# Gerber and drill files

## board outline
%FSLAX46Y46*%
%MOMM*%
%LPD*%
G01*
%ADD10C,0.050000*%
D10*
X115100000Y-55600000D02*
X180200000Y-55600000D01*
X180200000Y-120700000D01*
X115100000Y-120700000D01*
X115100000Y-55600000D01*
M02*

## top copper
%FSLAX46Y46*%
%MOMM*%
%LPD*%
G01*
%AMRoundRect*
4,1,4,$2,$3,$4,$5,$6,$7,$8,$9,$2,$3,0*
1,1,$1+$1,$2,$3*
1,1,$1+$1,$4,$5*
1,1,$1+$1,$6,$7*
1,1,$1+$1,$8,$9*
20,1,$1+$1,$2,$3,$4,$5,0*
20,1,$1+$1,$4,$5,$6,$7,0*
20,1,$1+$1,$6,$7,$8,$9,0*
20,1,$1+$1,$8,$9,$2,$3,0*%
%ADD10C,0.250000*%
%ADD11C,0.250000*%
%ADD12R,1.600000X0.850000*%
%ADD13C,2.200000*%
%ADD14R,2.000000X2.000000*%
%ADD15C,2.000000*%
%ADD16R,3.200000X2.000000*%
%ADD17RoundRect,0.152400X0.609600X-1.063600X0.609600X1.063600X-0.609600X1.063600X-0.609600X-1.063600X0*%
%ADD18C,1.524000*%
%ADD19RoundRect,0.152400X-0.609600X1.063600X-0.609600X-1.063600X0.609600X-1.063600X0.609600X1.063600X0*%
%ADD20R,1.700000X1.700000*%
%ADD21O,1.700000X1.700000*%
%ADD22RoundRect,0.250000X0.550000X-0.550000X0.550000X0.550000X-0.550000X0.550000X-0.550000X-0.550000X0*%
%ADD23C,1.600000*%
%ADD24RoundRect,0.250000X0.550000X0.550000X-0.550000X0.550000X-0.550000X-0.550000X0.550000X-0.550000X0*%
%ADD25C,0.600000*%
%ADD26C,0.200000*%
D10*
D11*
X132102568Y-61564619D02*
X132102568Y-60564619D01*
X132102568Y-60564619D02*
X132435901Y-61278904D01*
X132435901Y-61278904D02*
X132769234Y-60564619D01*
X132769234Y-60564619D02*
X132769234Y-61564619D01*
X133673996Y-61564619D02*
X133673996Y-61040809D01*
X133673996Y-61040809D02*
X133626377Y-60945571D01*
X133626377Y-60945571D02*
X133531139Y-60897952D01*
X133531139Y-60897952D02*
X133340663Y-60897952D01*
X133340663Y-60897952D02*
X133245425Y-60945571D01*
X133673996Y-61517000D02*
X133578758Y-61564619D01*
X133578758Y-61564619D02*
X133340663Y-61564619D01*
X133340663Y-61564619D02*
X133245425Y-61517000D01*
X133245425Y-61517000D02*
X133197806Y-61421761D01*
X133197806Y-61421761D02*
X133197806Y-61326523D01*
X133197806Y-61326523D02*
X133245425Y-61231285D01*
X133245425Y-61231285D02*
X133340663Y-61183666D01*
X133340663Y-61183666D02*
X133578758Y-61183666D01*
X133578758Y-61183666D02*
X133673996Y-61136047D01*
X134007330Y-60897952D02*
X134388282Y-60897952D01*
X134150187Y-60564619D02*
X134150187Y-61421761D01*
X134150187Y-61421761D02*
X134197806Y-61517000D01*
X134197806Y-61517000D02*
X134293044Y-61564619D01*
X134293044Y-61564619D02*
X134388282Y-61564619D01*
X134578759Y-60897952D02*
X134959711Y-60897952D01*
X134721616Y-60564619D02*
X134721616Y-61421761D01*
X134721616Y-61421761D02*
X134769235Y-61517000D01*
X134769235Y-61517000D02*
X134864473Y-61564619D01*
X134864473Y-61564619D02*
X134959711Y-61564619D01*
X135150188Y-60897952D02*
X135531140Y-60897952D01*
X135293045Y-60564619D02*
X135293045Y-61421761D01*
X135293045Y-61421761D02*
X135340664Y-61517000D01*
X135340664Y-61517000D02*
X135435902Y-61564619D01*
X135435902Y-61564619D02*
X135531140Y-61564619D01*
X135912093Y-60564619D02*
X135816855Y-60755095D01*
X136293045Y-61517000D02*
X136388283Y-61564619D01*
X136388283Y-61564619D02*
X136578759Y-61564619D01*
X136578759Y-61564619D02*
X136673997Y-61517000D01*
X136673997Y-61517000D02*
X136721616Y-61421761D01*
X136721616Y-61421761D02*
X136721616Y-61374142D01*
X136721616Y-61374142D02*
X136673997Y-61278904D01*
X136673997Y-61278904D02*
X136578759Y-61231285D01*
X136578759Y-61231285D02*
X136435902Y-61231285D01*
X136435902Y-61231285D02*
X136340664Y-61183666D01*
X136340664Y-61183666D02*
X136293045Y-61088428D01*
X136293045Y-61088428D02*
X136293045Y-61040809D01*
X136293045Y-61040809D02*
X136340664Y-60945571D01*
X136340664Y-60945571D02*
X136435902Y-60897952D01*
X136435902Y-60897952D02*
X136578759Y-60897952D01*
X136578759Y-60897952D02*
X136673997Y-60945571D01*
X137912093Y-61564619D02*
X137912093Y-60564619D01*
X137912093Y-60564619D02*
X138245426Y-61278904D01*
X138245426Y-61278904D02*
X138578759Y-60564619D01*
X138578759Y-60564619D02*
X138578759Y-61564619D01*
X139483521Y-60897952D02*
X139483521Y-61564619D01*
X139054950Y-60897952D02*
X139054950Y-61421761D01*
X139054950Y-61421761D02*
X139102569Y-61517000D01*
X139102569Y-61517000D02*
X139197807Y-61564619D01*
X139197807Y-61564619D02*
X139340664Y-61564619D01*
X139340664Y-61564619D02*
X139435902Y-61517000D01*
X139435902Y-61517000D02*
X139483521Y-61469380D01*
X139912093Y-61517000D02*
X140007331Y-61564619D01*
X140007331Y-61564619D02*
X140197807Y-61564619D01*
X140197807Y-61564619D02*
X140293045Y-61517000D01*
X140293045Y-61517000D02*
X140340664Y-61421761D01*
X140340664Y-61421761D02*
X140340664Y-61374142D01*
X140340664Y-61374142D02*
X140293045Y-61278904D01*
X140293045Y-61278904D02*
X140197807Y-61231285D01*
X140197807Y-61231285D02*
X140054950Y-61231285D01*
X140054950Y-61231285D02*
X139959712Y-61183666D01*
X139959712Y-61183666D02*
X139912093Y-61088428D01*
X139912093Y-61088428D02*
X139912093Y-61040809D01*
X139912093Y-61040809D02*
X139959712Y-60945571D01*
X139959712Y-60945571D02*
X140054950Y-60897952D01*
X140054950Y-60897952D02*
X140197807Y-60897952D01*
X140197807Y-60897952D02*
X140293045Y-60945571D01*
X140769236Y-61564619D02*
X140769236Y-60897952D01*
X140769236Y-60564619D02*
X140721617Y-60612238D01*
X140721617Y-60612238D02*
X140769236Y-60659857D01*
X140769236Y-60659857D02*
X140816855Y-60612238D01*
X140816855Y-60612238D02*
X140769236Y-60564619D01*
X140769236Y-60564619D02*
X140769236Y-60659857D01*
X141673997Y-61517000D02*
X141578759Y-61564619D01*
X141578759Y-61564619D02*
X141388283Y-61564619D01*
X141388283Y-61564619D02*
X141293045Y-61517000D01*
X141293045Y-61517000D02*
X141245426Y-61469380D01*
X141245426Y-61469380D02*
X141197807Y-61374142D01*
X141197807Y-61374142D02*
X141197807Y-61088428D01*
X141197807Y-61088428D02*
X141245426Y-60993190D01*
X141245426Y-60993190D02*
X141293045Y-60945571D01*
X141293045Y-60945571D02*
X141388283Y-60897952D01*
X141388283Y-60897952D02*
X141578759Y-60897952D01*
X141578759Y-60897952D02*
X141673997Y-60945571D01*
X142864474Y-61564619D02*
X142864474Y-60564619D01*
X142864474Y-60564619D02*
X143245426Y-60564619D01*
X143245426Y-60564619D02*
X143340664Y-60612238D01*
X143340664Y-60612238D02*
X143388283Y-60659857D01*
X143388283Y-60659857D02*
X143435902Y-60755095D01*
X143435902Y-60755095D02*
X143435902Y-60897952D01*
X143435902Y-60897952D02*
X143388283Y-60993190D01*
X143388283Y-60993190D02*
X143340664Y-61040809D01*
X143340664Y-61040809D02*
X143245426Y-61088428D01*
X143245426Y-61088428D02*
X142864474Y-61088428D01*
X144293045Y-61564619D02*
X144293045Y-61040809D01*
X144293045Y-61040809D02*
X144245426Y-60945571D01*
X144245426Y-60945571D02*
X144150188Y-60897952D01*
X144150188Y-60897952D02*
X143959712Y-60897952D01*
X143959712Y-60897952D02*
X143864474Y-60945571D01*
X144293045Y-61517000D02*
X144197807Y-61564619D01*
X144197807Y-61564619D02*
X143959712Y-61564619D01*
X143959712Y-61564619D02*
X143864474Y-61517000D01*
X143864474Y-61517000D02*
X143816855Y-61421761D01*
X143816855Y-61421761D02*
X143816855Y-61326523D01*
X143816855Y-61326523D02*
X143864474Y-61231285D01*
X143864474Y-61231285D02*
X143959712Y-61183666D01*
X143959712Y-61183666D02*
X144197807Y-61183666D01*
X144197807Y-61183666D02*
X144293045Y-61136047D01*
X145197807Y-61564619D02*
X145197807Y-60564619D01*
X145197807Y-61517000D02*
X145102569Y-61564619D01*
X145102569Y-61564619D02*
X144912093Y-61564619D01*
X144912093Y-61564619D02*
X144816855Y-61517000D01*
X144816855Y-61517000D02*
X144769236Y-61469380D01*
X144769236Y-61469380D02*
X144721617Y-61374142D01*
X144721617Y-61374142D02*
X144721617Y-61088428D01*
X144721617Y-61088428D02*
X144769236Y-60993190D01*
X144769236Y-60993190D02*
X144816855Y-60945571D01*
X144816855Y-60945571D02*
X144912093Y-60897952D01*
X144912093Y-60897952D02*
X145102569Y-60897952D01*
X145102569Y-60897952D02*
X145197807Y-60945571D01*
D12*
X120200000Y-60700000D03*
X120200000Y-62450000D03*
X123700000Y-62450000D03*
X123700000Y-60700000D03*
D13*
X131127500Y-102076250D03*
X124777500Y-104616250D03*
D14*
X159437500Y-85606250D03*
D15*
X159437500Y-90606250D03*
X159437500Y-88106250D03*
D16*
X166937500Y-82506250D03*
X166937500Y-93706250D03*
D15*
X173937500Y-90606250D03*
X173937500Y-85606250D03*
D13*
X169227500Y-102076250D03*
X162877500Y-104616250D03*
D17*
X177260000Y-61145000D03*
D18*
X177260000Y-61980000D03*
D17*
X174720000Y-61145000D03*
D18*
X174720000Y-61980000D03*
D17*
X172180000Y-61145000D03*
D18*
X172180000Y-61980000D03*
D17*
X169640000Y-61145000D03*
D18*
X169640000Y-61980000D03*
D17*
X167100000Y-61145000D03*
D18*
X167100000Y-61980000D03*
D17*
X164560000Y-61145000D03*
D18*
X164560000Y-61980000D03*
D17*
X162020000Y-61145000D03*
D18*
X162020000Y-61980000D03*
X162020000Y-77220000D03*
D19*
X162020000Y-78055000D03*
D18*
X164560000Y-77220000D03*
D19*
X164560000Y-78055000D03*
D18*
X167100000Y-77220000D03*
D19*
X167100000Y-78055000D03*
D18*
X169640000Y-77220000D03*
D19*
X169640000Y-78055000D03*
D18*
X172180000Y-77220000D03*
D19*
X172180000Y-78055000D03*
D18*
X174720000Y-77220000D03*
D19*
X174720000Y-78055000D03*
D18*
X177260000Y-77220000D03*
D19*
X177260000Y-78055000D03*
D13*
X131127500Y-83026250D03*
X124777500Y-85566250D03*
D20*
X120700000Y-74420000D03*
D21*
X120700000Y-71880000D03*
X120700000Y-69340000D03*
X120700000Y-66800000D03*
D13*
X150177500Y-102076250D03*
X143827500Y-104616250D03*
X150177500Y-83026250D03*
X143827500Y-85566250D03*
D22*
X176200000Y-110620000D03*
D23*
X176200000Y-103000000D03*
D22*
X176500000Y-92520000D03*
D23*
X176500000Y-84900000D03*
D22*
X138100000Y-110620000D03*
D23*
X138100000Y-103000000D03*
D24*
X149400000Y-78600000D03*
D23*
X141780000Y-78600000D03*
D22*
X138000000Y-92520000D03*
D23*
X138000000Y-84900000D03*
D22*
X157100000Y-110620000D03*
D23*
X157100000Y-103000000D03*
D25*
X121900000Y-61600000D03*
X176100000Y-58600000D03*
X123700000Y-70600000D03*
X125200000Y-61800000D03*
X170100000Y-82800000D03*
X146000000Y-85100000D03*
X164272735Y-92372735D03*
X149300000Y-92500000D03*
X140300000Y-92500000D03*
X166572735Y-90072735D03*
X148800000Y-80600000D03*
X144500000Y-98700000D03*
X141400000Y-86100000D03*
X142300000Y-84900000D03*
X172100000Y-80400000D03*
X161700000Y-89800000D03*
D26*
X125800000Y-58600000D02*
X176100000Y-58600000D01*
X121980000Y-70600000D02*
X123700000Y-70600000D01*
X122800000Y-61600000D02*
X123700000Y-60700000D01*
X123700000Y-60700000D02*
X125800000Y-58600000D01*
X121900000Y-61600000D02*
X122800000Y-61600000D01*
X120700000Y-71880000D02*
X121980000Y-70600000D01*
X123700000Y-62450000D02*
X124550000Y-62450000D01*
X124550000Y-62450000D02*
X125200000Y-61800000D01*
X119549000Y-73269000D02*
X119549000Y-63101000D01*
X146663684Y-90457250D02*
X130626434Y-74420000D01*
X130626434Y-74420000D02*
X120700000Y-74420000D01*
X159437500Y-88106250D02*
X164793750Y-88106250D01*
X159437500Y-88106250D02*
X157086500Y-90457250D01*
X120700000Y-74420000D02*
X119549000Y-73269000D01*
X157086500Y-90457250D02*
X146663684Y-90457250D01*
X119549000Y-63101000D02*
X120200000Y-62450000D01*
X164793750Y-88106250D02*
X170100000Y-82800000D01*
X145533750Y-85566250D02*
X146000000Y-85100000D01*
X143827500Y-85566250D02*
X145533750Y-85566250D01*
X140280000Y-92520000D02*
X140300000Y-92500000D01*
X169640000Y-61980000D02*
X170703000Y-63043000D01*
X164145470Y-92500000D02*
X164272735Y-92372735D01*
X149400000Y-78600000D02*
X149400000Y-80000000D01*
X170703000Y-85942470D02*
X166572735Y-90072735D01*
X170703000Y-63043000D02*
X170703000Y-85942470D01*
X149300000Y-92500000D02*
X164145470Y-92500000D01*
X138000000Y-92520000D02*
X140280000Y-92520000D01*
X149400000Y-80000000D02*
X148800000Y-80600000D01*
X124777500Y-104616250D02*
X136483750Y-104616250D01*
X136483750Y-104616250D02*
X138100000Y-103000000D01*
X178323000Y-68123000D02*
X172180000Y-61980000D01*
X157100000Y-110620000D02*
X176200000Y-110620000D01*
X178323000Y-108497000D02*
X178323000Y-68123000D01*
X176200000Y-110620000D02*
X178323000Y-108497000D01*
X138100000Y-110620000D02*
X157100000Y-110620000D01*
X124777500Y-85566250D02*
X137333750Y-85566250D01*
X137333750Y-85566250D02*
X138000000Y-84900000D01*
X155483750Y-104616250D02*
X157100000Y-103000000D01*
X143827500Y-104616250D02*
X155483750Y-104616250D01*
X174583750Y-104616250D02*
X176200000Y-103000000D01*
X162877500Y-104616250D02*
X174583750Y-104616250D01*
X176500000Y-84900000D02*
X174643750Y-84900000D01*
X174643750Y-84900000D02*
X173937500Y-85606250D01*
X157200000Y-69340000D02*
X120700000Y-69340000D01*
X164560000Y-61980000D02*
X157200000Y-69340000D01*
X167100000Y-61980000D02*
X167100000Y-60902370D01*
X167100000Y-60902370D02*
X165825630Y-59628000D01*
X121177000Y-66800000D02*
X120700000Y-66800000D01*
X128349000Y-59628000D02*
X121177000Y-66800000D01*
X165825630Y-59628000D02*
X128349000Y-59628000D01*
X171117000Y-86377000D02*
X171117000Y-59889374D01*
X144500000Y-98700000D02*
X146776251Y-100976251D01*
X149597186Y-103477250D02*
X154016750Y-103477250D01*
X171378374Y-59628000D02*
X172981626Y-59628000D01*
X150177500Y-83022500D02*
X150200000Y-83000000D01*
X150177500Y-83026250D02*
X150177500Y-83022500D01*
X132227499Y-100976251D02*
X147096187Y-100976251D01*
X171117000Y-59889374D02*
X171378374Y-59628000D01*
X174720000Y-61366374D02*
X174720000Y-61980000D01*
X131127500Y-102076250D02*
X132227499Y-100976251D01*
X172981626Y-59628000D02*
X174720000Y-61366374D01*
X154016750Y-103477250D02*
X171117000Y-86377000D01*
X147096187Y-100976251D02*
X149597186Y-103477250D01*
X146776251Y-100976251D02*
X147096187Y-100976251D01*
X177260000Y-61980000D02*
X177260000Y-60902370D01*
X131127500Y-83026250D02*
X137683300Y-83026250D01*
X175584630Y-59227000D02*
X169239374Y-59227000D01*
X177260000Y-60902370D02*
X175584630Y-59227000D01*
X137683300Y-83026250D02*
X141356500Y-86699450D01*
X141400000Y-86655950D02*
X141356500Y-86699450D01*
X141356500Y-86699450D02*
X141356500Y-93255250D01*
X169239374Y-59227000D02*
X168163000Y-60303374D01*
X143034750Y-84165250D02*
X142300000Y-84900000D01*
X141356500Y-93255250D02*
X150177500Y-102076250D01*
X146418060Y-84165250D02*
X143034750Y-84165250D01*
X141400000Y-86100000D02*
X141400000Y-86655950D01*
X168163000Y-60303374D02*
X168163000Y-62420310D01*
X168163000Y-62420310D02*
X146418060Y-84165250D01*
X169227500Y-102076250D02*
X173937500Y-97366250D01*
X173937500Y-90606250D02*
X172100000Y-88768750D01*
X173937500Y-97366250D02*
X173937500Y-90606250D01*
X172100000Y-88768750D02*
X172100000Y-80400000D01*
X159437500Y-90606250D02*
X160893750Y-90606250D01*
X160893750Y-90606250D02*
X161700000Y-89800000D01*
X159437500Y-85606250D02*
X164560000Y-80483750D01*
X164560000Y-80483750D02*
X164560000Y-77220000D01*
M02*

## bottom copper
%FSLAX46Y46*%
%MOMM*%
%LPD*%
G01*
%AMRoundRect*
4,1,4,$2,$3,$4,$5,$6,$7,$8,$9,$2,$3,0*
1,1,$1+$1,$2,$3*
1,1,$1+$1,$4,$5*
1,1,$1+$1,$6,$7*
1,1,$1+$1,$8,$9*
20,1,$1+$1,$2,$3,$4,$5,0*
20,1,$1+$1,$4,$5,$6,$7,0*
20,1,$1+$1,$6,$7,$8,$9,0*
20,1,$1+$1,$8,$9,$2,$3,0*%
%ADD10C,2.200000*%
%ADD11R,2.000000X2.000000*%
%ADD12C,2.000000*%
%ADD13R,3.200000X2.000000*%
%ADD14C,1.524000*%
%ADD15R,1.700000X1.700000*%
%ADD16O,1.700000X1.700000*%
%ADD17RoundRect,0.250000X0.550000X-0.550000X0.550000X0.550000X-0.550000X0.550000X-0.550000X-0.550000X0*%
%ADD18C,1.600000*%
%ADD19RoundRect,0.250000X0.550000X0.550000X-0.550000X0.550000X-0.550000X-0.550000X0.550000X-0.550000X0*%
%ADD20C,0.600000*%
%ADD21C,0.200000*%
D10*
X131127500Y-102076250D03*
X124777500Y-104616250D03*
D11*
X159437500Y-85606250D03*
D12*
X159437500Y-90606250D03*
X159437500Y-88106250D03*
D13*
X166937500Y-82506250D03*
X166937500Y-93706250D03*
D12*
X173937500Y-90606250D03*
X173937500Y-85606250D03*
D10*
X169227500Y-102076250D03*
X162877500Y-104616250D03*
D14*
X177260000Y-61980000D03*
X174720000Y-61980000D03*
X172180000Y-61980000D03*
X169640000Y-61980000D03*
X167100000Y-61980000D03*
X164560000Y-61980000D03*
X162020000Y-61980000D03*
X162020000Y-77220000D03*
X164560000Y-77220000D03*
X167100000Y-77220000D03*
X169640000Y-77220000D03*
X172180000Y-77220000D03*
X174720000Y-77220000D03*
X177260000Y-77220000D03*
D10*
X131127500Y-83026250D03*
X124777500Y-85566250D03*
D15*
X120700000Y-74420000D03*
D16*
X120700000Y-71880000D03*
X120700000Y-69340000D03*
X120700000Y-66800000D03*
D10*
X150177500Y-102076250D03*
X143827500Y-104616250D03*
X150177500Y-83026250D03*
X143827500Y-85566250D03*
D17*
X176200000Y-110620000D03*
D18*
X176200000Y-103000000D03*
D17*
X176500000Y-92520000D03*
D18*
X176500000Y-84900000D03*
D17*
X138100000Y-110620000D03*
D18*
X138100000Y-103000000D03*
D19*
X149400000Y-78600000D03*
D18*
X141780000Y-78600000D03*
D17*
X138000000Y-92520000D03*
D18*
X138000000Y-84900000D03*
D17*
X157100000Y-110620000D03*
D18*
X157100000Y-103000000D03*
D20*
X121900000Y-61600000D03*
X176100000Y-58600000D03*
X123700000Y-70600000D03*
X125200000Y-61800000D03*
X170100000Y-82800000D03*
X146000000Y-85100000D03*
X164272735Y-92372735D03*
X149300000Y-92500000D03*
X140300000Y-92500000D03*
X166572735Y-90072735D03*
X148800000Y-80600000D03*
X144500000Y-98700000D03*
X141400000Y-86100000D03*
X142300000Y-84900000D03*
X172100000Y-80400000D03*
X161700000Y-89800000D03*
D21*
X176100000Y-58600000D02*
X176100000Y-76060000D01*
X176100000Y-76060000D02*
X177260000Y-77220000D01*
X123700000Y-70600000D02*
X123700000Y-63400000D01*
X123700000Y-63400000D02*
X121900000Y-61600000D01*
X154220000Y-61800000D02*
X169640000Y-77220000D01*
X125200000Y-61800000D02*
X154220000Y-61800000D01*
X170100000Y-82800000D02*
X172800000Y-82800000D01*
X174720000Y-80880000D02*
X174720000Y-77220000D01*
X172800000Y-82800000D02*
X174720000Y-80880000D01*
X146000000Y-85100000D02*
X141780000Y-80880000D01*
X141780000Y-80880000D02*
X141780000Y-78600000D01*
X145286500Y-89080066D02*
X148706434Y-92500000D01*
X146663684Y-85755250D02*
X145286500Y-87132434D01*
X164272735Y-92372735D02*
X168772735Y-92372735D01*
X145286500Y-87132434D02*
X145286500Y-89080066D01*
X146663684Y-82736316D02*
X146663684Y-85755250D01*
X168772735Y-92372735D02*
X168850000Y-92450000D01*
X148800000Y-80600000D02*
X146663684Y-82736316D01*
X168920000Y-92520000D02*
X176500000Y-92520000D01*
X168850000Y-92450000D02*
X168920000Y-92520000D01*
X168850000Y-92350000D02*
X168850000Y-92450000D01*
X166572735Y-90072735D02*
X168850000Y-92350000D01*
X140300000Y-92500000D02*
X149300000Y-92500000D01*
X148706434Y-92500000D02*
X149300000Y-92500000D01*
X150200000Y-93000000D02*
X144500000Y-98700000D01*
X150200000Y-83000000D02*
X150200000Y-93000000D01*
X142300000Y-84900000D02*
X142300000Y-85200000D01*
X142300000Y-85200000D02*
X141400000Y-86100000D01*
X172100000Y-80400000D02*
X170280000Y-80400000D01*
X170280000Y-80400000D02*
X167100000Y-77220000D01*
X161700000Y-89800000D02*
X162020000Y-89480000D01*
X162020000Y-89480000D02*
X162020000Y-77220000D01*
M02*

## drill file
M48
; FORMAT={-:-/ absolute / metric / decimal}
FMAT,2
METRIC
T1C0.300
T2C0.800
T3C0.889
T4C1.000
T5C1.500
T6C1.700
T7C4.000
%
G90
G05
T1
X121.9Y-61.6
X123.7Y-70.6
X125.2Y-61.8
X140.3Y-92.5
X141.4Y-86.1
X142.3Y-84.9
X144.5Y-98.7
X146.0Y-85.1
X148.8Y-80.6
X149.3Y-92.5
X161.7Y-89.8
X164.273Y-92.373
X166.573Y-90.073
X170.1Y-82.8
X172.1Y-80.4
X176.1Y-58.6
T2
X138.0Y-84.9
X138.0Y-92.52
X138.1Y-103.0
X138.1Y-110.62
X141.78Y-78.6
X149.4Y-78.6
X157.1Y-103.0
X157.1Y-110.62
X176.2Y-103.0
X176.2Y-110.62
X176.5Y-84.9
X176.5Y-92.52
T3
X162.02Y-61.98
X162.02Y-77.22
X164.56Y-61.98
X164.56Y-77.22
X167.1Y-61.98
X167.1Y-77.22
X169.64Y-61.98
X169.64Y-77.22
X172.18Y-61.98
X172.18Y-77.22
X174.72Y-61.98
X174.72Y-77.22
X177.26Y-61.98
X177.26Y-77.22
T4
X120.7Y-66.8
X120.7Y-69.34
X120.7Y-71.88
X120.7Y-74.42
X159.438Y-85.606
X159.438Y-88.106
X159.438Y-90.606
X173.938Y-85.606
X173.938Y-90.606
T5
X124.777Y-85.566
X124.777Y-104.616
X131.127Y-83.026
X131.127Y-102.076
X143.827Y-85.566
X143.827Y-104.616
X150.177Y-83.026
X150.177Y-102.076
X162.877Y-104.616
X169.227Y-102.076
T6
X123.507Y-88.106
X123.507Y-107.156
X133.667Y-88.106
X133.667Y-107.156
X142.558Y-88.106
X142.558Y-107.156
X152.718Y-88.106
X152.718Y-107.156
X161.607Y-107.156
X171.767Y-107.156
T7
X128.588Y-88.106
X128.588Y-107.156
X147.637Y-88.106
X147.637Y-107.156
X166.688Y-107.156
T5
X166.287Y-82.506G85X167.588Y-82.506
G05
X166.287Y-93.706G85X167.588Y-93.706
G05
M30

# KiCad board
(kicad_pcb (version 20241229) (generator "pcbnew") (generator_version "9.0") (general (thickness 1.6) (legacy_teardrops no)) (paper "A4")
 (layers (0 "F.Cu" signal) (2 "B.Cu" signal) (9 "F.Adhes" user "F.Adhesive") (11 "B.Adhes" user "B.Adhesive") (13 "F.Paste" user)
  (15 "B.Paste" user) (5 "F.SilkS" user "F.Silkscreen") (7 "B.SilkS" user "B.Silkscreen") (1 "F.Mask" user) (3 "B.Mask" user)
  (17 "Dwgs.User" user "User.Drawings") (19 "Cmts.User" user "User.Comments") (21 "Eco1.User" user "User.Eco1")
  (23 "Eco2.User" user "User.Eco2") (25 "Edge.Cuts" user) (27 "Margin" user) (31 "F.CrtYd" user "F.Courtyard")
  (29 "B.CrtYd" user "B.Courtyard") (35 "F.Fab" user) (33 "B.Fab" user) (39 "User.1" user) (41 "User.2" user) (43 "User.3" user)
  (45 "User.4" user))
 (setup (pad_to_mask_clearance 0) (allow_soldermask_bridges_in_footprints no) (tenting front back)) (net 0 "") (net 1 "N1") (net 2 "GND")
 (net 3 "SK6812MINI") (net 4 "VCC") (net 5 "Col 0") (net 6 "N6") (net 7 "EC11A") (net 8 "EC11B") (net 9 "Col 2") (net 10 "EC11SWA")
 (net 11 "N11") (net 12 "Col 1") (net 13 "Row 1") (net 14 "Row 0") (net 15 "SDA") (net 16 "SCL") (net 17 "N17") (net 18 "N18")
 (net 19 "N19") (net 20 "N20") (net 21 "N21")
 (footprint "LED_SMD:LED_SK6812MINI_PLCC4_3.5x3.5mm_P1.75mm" (layer "F.Cu") (at 121.95 61.575)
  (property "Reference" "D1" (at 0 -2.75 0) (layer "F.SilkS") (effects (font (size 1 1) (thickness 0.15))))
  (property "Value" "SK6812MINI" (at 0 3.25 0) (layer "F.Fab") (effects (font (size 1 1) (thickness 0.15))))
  (pad "1" smd rect (at -1.75 -0.875) (size 1.6 0.85) (layers "F.Cu" "F.Mask" "F.Paste") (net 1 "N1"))
  (pad "2" smd rect (at -1.75 0.875) (size 1.6 0.85) (layers "F.Cu" "F.Mask" "F.Paste") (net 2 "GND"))
  (pad "3" smd rect (at 1.75 0.875) (size 1.6 0.85) (layers "F.Cu" "F.Mask" "F.Paste") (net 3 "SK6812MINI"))
  (pad "4" smd rect (at 1.75 -0.875) (size 1.6 0.85) (layers "F.Cu" "F.Mask" "F.Paste") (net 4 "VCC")))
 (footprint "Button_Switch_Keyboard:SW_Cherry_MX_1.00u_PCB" (layer "F.Cu") (at 131.1275 102.07625)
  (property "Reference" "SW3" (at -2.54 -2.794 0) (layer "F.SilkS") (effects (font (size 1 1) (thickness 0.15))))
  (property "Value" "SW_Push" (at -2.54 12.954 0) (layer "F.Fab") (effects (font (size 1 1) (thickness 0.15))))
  (pad "" np_thru_hole circle (at -7.62 5.08) (size 1.7 1.7) (drill 1.7) (layers "*.Cu" "*.Mask"))
  (pad "" np_thru_hole circle (at -2.54 5.08) (size 4 4) (drill 4) (layers "*.Cu" "*.Mask"))
  (pad "" np_thru_hole circle (at 2.54 5.08) (size 1.7 1.7) (drill 1.7) (layers "*.Cu" "*.Mask"))
  (pad "1" thru_hole circle (at 0 0) (size 2.2 2.2) (drill 1.5) (layers "*.Cu" "*.Mask") (remove_unused_layers no) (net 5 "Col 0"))
  (pad "2" thru_hole circle (at -6.35 2.54) (size 2.2 2.2) (drill 1.5) (layers "*.Cu" "*.Mask") (remove_unused_layers no) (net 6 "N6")))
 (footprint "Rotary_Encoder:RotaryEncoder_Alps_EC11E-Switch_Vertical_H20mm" (layer "F.Cu") (at 159.4375 85.60625)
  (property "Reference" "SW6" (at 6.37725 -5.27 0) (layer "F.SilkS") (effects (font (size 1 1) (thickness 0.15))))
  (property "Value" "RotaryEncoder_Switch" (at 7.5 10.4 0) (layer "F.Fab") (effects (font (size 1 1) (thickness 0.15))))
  (pad "A" thru_hole rect (at 0 0) (size 2 2) (drill 1) (layers "*.Cu" "*.Mask") (remove_unused_layers no) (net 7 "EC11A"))
  (pad "B" thru_hole circle (at 0 5) (size 2 2) (drill 1) (layers "*.Cu" "*.Mask") (remove_unused_layers no) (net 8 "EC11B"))
  (pad "C" thru_hole circle (at 0 2.5) (size 2 2) (drill 1) (layers "*.Cu" "*.Mask") (remove_unused_layers no) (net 2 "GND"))
  (pad "MP" thru_hole rect (at 7.5 -3.1) (size 3.2 2) (drill oval 2.8 1.5) (layers "*.Cu" "*.Mask") (remove_unused_layers no))
  (pad "MP" thru_hole rect (at 7.5 8.1) (size 3.2 2) (drill oval 2.8 1.5) (layers "*.Cu" "*.Mask") (remove_unused_layers no))
  (pad "S1" thru_hole circle (at 14.5 5) (size 2 2) (drill 1) (layers "*.Cu" "*.Mask") (remove_unused_layers no) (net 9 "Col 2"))
  (pad "S2" thru_hole circle (at 14.5 0) (size 2 2) (drill 1) (layers "*.Cu" "*.Mask") (remove_unused_layers no) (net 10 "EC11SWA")))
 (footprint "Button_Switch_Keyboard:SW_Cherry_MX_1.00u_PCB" (layer "F.Cu") (at 169.2275 102.07625)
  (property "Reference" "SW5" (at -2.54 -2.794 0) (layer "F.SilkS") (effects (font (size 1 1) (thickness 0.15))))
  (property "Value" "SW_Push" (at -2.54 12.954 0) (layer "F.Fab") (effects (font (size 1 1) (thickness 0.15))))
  (pad "" np_thru_hole circle (at -7.62 5.08) (size 1.7 1.7) (drill 1.7) (layers "*.Cu" "*.Mask"))
  (pad "" np_thru_hole circle (at -2.54 5.08) (size 4 4) (drill 4) (layers "*.Cu" "*.Mask"))
  (pad "" np_thru_hole circle (at 2.54 5.08) (size 1.7 1.7) (drill 1.7) (layers "*.Cu" "*.Mask"))
  (pad "1" thru_hole circle (at 0 0) (size 2.2 2.2) (drill 1.5) (layers "*.Cu" "*.Mask") (remove_unused_layers no) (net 9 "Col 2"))
  (pad "2" thru_hole circle (at -6.35 2.54) (size 2.2 2.2) (drill 1.5) (layers "*.Cu" "*.Mask") (remove_unused_layers no) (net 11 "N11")))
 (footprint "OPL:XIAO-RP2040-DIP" (layer "F.Cu") (at 169.64 69.6 -90)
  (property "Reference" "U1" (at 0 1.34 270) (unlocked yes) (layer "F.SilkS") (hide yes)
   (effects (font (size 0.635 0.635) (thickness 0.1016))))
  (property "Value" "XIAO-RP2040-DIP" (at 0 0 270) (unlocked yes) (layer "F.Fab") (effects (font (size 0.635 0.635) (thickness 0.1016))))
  (pad "1" smd roundrect (at -8.455 -7.62 90) (size 2.432 1.524) (layers "F.Cu" "F.Mask") (roundrect_rratio 0.1) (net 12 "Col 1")
   (thermal_bridge_angle 45))
  (pad "1" thru_hole circle (at -7.62 -7.62 90) (size 1.524 1.524) (drill 0.889) (layers "*.Cu" "*.Mask") (remove_unused_layers no)
   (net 12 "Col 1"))
  (pad "2" smd roundrect (at -8.455 -5.08 90) (size 2.432 1.524) (layers "F.Cu" "F.Mask") (roundrect_rratio 0.1) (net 5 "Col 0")
   (thermal_bridge_angle 45))
  (pad "2" thru_hole circle (at -7.62 -5.08 90) (size 1.524 1.524) (drill 0.889) (layers "*.Cu" "*.Mask") (remove_unused_layers no)
   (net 5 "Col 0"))
  (pad "3" smd roundrect (at -8.455 -2.54 90) (size 2.432 1.524) (layers "F.Cu" "F.Mask") (roundrect_rratio 0.1) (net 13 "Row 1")
   (thermal_bridge_angle 45))
  (pad "3" thru_hole circle (at -7.62 -2.54 90) (size 1.524 1.524) (drill 0.889) (layers "*.Cu" "*.Mask") (remove_unused_layers no)
   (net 13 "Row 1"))
  (pad "4" smd roundrect (at -8.455 0 90) (size 2.432 1.524) (layers "F.Cu" "F.Mask") (roundrect_rratio 0.1) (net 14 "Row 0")
   (thermal_bridge_angle 45))
  (pad "4" thru_hole circle (at -7.62 0 90) (size 1.524 1.524) (drill 0.889) (layers "*.Cu" "*.Mask") (remove_unused_layers no)
   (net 14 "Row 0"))
  (pad "5" smd roundrect (at -8.455 2.54 90) (size 2.432 1.524) (layers "F.Cu" "F.Mask") (roundrect_rratio 0.1) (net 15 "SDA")
   (thermal_bridge_angle 45))
  (pad "5" thru_hole circle (at -7.62 2.54 90) (size 1.524 1.524) (drill 0.889) (layers "*.Cu" "*.Mask") (remove_unused_layers no)
   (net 15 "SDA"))
  (pad "6" smd roundrect (at -8.455 5.08 90) (size 2.432 1.524) (layers "F.Cu" "F.Mask") (roundrect_rratio 0.1) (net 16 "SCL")
   (thermal_bridge_angle 45))
  (pad "6" thru_hole circle (at -7.62 5.08 90) (size 1.524 1.524) (drill 0.889) (layers "*.Cu" "*.Mask") (remove_unused_layers no)
   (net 16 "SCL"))
  (pad "7" smd roundrect (at -8.455 7.62 90) (size 2.432 1.524) (layers "F.Cu" "F.Mask") (roundrect_rratio 0.1) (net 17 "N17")
   (thermal_bridge_angle 45))
  (pad "7" thru_hole circle (at -7.62 7.62 90) (size 1.524 1.524) (drill 0.889) (layers "*.Cu" "*.Mask") (remove_unused_layers no)
   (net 17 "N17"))
  (pad "8" thru_hole circle (at 7.62 7.62 270) (size 1.524 1.524) (drill 0.889) (layers "*.Cu" "*.Mask") (remove_unused_layers no)
   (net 8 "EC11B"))
  (pad "8" smd roundrect (at 8.455 7.62 270) (size 2.432 1.524) (layers "F.Cu" "F.Mask") (roundrect_rratio 0.1) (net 8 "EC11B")
   (thermal_bridge_angle 45))
  (pad "9" thru_hole circle (at 7.62 5.08 270) (size 1.524 1.524) (drill 0.889) (layers "*.Cu" "*.Mask") (remove_unused_layers no)
   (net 7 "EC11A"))
  (pad "9" smd roundrect (at 8.455 5.08 270) (size 2.432 1.524) (layers "F.Cu" "F.Mask") (roundrect_rratio 0.1) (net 7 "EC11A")
   (thermal_bridge_angle 45))
  (pad "10" thru_hole circle (at 7.62 2.54 270) (size 1.524 1.524) (drill 0.889) (layers "*.Cu" "*.Mask") (remove_unused_layers no)
   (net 9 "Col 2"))
  (pad "10" smd roundrect (at 8.455 2.54 270) (size 2.432 1.524) (layers "F.Cu" "F.Mask") (roundrect_rratio 0.1) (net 9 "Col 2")
   (thermal_bridge_angle 45))
  (pad "11" thru_hole circle (at 7.62 0 270) (size 1.524 1.524) (drill 0.889) (layers "*.Cu" "*.Mask") (remove_unused_layers no)
   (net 3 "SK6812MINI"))
  (pad "11" smd roundrect (at 8.455 0 270) (size 2.432 1.524) (layers "F.Cu" "F.Mask") (roundrect_rratio 0.1) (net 3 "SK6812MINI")
   (thermal_bridge_angle 45))
  (pad "12" thru_hole circle (at 7.62 -2.54 270) (size 1.524 1.524) (drill 0.889) (layers "*.Cu" "*.Mask") (remove_unused_layers no)
   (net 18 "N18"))
  (pad "12" smd roundrect (at 8.455 -2.54 270) (size 2.432 1.524) (layers "F.Cu" "F.Mask") (roundrect_rratio 0.1) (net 18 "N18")
   (thermal_bridge_angle 45))
  (pad "13" thru_hole circle (at 7.62 -5.08 270) (size 1.524 1.524) (drill 0.889) (layers "*.Cu" "*.Mask") (remove_unused_layers no)
   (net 2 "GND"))
  (pad "13" smd roundrect (at 8.455 -5.08 270) (size 2.432 1.524) (layers "F.Cu" "F.Mask") (roundrect_rratio 0.1) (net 2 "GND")
   (thermal_bridge_angle 45))
  (pad "14" thru_hole circle (at 7.62 -7.62 270) (size 1.524 1.524) (drill 0.889) (layers "*.Cu" "*.Mask") (remove_unused_layers no)
   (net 4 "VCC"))
  (pad "14" smd roundrect (at 8.455 -7.62 270) (size 2.432 1.524) (layers "F.Cu" "F.Mask") (roundrect_rratio 0.1) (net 4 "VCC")
   (thermal_bridge_angle 45)))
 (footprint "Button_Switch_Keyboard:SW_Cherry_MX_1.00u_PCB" (layer "F.Cu") (at 131.1275 83.02625)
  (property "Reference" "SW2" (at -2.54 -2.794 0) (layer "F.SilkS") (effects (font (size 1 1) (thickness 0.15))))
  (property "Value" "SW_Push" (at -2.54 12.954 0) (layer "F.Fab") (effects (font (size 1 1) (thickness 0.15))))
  (pad "" np_thru_hole circle (at -7.62 5.08) (size 1.7 1.7) (drill 1.7) (layers "*.Cu" "*.Mask"))
  (pad "" np_thru_hole circle (at -2.54 5.08) (size 4 4) (drill 4) (layers "*.Cu" "*.Mask"))
  (pad "" np_thru_hole circle (at 2.54 5.08) (size 1.7 1.7) (drill 1.7) (layers "*.Cu" "*.Mask"))
  (pad "1" thru_hole circle (at 0 0) (size 2.2 2.2) (drill 1.5) (layers "*.Cu" "*.Mask") (remove_unused_layers no) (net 12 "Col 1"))
  (pad "2" thru_hole circle (at -6.35 2.54) (size 2.2 2.2) (drill 1.5) (layers "*.Cu" "*.Mask") (remove_unused_layers no) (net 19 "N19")))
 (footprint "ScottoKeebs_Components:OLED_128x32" (layer "F.Cu") (at 119.1 64.62)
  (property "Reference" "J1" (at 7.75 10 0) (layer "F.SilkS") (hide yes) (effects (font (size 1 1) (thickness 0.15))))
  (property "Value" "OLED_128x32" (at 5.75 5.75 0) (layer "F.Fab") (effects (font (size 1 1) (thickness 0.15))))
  (pad "1" thru_hole rect (at 1.6 9.8 180) (size 1.7 1.7) (drill 1) (layers "*.Cu" "*.Mask") (remove_unused_layers no) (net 2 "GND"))
  (pad "2" thru_hole oval (at 1.6 7.26 180) (size 1.7 1.7) (drill 1) (layers "*.Cu" "*.Mask") (remove_unused_layers no) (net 4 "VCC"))
  (pad "3" thru_hole oval (at 1.6 4.72 180) (size 1.7 1.7) (drill 1) (layers "*.Cu" "*.Mask") (remove_unused_layers no) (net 16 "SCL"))
  (pad "4" thru_hole oval (at 1.6 2.18 180) (size 1.7 1.7) (drill 1) (layers "*.Cu" "*.Mask") (remove_unused_layers no) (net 15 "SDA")))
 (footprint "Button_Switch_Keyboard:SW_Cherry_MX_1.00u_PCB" (layer "F.Cu") (at 150.1775 102.07625)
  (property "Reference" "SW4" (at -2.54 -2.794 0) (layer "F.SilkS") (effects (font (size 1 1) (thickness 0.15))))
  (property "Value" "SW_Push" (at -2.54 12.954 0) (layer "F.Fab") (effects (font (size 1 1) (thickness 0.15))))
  (pad "" np_thru_hole circle (at -7.62 5.08) (size 1.7 1.7) (drill 1.7) (layers "*.Cu" "*.Mask"))
  (pad "" np_thru_hole circle (at -2.54 5.08) (size 4 4) (drill 4) (layers "*.Cu" "*.Mask"))
  (pad "" np_thru_hole circle (at 2.54 5.08) (size 1.7 1.7) (drill 1.7) (layers "*.Cu" "*.Mask"))
  (pad "1" thru_hole circle (at 0 0) (size 2.2 2.2) (drill 1.5) (layers "*.Cu" "*.Mask") (remove_unused_layers no) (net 12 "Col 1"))
  (pad "2" thru_hole circle (at -6.35 2.54) (size 2.2 2.2) (drill 1.5) (layers "*.Cu" "*.Mask") (remove_unused_layers no) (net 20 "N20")))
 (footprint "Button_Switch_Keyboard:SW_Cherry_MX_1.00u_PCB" (layer "F.Cu") (at 150.1775 83.02625)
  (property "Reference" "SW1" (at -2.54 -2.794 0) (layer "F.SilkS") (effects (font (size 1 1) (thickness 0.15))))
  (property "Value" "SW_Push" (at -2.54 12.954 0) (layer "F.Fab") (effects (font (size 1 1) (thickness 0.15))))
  (pad "" np_thru_hole circle (at -7.62 5.08) (size 1.7 1.7) (drill 1.7) (layers "*.Cu" "*.Mask"))
  (pad "" np_thru_hole circle (at -2.54 5.08) (size 4 4) (drill 4) (layers "*.Cu" "*.Mask"))
  (pad "" np_thru_hole circle (at 2.54 5.08) (size 1.7 1.7) (drill 1.7) (layers "*.Cu" "*.Mask"))
  (pad "1" thru_hole circle (at 0 0) (size 2.2 2.2) (drill 1.5) (layers "*.Cu" "*.Mask") (remove_unused_layers no) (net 5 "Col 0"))
  (pad "2" thru_hole circle (at -6.35 2.54) (size 2.2 2.2) (drill 1.5) (layers "*.Cu" "*.Mask") (remove_unused_layers no) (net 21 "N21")))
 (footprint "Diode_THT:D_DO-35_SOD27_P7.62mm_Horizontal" (layer "B.Cu") (at 176.2 110.62 90)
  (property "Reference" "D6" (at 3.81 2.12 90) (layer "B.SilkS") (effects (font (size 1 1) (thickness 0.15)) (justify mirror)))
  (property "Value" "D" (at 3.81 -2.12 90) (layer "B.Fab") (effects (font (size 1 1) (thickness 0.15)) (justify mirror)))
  (pad "1" thru_hole roundrect (at 0 0 90) (size 1.6 1.6) (drill 0.8) (layers "*.Cu" "*.Mask") (remove_unused_layers no)
   (roundrect_rratio 0.15625) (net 13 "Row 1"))
  (pad "2" thru_hole circle (at 7.62 0 90) (size 1.6 1.6) (drill 0.8) (layers "*.Cu" "*.Mask") (remove_unused_layers no) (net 11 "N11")))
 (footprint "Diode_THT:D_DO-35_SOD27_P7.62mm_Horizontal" (layer "B.Cu") (at 176.5 92.52 90)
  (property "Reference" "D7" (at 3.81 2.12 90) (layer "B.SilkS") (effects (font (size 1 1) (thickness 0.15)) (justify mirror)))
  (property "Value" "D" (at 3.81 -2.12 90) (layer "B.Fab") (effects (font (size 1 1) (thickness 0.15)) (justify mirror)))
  (pad "1" thru_hole roundrect (at 0 0 90) (size 1.6 1.6) (drill 0.8) (layers "*.Cu" "*.Mask") (remove_unused_layers no)
   (roundrect_rratio 0.15625) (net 14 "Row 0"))
  (pad "2" thru_hole circle (at 7.62 0 90) (size 1.6 1.6) (drill 0.8) (layers "*.Cu" "*.Mask") (remove_unused_layers no) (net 10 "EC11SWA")))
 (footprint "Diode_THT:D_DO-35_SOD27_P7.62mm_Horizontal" (layer "B.Cu") (at 138.1 110.62 90)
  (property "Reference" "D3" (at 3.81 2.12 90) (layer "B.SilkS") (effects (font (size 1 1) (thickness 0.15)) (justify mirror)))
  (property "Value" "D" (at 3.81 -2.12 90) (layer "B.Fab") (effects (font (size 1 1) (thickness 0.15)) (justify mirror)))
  (pad "1" thru_hole roundrect (at 0 0 90) (size 1.6 1.6) (drill 0.8) (layers "*.Cu" "*.Mask") (remove_unused_layers no)
   (roundrect_rratio 0.15625) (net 13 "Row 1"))
  (pad "2" thru_hole circle (at 7.62 0 90) (size 1.6 1.6) (drill 0.8) (layers "*.Cu" "*.Mask") (remove_unused_layers no) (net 6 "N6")))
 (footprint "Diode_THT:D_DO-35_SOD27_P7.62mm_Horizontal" (layer "B.Cu") (at 149.4 78.6 180)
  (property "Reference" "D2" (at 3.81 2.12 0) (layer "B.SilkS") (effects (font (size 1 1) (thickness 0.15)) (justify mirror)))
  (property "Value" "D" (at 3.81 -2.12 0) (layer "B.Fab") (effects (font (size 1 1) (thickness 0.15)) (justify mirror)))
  (pad "1" thru_hole roundrect (at 0 0 180) (size 1.6 1.6) (drill 0.8) (layers "*.Cu" "*.Mask") (remove_unused_layers no)
   (roundrect_rratio 0.15625) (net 14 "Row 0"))
  (pad "2" thru_hole circle (at 7.62 0 180) (size 1.6 1.6) (drill 0.8) (layers "*.Cu" "*.Mask") (remove_unused_layers no) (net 21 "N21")))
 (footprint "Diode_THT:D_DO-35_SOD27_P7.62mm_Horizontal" (layer "B.Cu") (at 138 92.52 90)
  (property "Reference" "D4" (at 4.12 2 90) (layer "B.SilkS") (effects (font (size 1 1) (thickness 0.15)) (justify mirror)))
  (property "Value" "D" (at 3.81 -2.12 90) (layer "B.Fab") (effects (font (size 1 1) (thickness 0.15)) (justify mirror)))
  (pad "1" thru_hole roundrect (at 0 0 90) (size 1.6 1.6) (drill 0.8) (layers "*.Cu" "*.Mask") (remove_unused_layers no)
   (roundrect_rratio 0.15625) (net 14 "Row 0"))
  (pad "2" thru_hole circle (at 7.62 0 90) (size 1.6 1.6) (drill 0.8) (layers "*.Cu" "*.Mask") (remove_unused_layers no) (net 19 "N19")))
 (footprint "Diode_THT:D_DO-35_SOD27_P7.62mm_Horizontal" (layer "B.Cu") (at 157.1 110.62 90)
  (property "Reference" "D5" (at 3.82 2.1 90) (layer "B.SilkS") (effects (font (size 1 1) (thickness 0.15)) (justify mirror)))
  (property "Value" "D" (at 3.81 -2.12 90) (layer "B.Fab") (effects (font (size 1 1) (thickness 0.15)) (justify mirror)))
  (pad "1" thru_hole roundrect (at 0 0 90) (size 1.6 1.6) (drill 0.8) (layers "*.Cu" "*.Mask") (remove_unused_layers no)
   (roundrect_rratio 0.15625) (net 13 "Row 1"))
  (pad "2" thru_hole circle (at 7.62 0 90) (size 1.6 1.6) (drill 0.8) (layers "*.Cu" "*.Mask") (remove_unused_layers no) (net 20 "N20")))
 (gr_rect (start 115.1 55.6) (end 180.2 120.7) (stroke (width 0.05) (type default)) (fill no) (layer "Edge.Cuts"))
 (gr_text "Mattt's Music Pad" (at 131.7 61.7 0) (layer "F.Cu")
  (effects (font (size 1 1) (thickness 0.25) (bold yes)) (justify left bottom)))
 (segment (start 125.8 58.6) (end 176.1 58.6) (width 0.2) (layer "F.Cu") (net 4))
 (segment (start 121.98 70.6) (end 123.7 70.6) (width 0.2) (layer "F.Cu") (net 4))
 (segment (start 122.8 61.6) (end 123.7 60.7) (width 0.2) (layer "F.Cu") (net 4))
 (segment (start 123.7 60.7) (end 125.8 58.6) (width 0.2) (layer "F.Cu") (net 4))
 (segment (start 121.9 61.6) (end 122.8 61.6) (width 0.2) (layer "F.Cu") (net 4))
 (segment (start 120.7 71.88) (end 121.98 70.6) (width 0.2) (layer "F.Cu") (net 4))
 (via (at 121.9 61.6) (size 0.6) (drill 0.3) (layers "F.Cu" "B.Cu") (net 4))
 (via (at 176.1 58.6) (size 0.6) (drill 0.3) (layers "F.Cu" "B.Cu") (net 4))
 (via (at 123.7 70.6) (size 0.6) (drill 0.3) (layers "F.Cu" "B.Cu") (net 4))
 (segment (start 176.1 58.6) (end 176.1 76.06) (width 0.2) (layer "B.Cu") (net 4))
 (segment (start 176.1 76.06) (end 177.26 77.22) (width 0.2) (layer "B.Cu") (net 4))
 (segment (start 123.7 70.6) (end 123.7 63.4) (width 0.2) (layer "B.Cu") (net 4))
 (segment (start 123.7 63.4) (end 121.9 61.6) (width 0.2) (layer "B.Cu") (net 4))
 (segment (start 123.7 62.45) (end 124.55 62.45) (width 0.2) (layer "F.Cu") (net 3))
 (segment (start 124.55 62.45) (end 125.2 61.8) (width 0.2) (layer "F.Cu") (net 3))
 (via (at 125.2 61.8) (size 0.6) (drill 0.3) (layers "F.Cu" "B.Cu") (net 3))
 (segment (start 154.22 61.8) (end 169.64 77.22) (width 0.2) (layer "B.Cu") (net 3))
 (segment (start 125.2 61.8) (end 154.22 61.8) (width 0.2) (layer "B.Cu") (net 3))
 (segment (start 119.549 73.269) (end 119.549 63.101) (width 0.2) (layer "F.Cu") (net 2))
 (segment (start 146.663684 90.45725) (end 130.626434 74.42) (width 0.2) (layer "F.Cu") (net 2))
 (segment (start 130.626434 74.42) (end 120.7 74.42) (width 0.2) (layer "F.Cu") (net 2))
 (segment (start 159.4375 88.10625) (end 164.79375 88.10625) (width 0.2) (layer "F.Cu") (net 2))
 (segment (start 159.4375 88.10625) (end 157.0865 90.45725) (width 0.2) (layer "F.Cu") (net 2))
 (segment (start 120.7 74.42) (end 119.549 73.269) (width 0.2) (layer "F.Cu") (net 2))
 (segment (start 157.0865 90.45725) (end 146.663684 90.45725) (width 0.2) (layer "F.Cu") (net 2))
 (segment (start 119.549 63.101) (end 120.2 62.45) (width 0.2) (layer "F.Cu") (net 2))
 (segment (start 164.79375 88.10625) (end 170.1 82.8) (width 0.2) (layer "F.Cu") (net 2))
 (via (at 170.1 82.8) (size 0.6) (drill 0.3) (layers "F.Cu" "B.Cu") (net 2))
 (segment (start 170.1 82.8) (end 172.8 82.8) (width 0.2) (layer "B.Cu") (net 2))
 (segment (start 174.72 80.88) (end 174.72 77.22) (width 0.2) (layer "B.Cu") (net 2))
 (segment (start 172.8 82.8) (end 174.72 80.88) (width 0.2) (layer "B.Cu") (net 2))
 (segment (start 145.53375 85.56625) (end 146 85.1) (width 0.2) (layer "F.Cu") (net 21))
 (segment (start 143.8275 85.56625) (end 145.53375 85.56625) (width 0.2) (layer "F.Cu") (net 21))
 (via (at 146 85.1) (size 0.6) (drill 0.3) (layers "F.Cu" "B.Cu") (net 21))
 (segment (start 146 85.1) (end 141.78 80.88) (width 0.2) (layer "B.Cu") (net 21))
 (segment (start 141.78 80.88) (end 141.78 78.6) (width 0.2) (layer "B.Cu") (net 21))
 (segment (start 140.28 92.52) (end 140.3 92.5) (width 0.2) (layer "F.Cu") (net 14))
 (segment (start 169.64 61.98) (end 170.703 63.043) (width 0.2) (layer "F.Cu") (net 14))
 (segment (start 164.14547 92.5) (end 164.272735 92.372735) (width 0.2) (layer "F.Cu") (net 14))
 (segment (start 149.4 78.6) (end 149.4 80) (width 0.2) (layer "F.Cu") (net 14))
 (segment (start 170.703 85.94247) (end 166.572735 90.072735) (width 0.2) (layer "F.Cu") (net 14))
 (segment (start 170.703 63.043) (end 170.703 85.94247) (width 0.2) (layer "F.Cu") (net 14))
 (segment (start 149.3 92.5) (end 164.14547 92.5) (width 0.2) (layer "F.Cu") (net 14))
 (segment (start 138 92.52) (end 140.28 92.52) (width 0.2) (layer "F.Cu") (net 14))
 (segment (start 149.4 80) (end 148.8 80.6) (width 0.2) (layer "F.Cu") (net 14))
 (via (at 164.272735 92.372735) (size 0.6) (drill 0.3) (layers "F.Cu" "B.Cu") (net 14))
 (via (at 149.3 92.5) (size 0.6) (drill 0.3) (layers "F.Cu" "B.Cu") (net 14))
 (via (at 140.3 92.5) (size 0.6) (drill 0.3) (layers "F.Cu" "B.Cu") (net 14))
 (via (at 166.572735 90.072735) (size 0.6) (drill 0.3) (layers "F.Cu" "B.Cu") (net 14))
 (via (at 148.8 80.6) (size 0.6) (drill 0.3) (layers "F.Cu" "B.Cu") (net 14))
 (segment (start 145.2865 89.080066) (end 148.706434 92.5) (width 0.2) (layer "B.Cu") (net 14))
 (segment (start 146.663684 85.75525) (end 145.2865 87.132434) (width 0.2) (layer "B.Cu") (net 14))
 (segment (start 164.272735 92.372735) (end 168.772735 92.372735) (width 0.2) (layer "B.Cu") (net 14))
 (segment (start 145.2865 87.132434) (end 145.2865 89.080066) (width 0.2) (layer "B.Cu") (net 14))
 (segment (start 146.663684 82.736316) (end 146.663684 85.75525) (width 0.2) (layer "B.Cu") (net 14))
 (segment (start 168.772735 92.372735) (end 168.85 92.45) (width 0.2) (layer "B.Cu") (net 14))
 (segment (start 148.8 80.6) (end 146.663684 82.736316) (width 0.2) (layer "B.Cu") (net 14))
 (segment (start 168.92 92.52) (end 176.5 92.52) (width 0.2) (layer "B.Cu") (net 14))
 (segment (start 168.85 92.45) (end 168.92 92.52) (width 0.2) (layer "B.Cu") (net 14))
 (segment (start 168.85 92.35) (end 168.85 92.45) (width 0.2) (layer "B.Cu") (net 14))
 (segment (start 166.572735 90.072735) (end 168.85 92.35) (width 0.2) (layer "B.Cu") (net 14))
 (segment (start 140.3 92.5) (end 149.3 92.5) (width 0.2) (layer "B.Cu") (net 14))
 (segment (start 148.706434 92.5) (end 149.3 92.5) (width 0.2) (layer "B.Cu") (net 14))
 (segment (start 124.7775 104.61625) (end 136.48375 104.61625) (width 0.2) (layer "F.Cu") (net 6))
 (segment (start 136.48375 104.61625) (end 138.1 103) (width 0.2) (layer "F.Cu") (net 6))
 (segment (start 178.323 68.123) (end 172.18 61.98) (width 0.2) (layer "F.Cu") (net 13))
 (segment (start 157.1 110.62) (end 176.2 110.62) (width 0.2) (layer "F.Cu") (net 13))
 (segment (start 178.323 108.497) (end 178.323 68.123) (width 0.2) (layer "F.Cu") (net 13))
 (segment (start 176.2 110.62) (end 178.323 108.497) (width 0.2) (layer "F.Cu") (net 13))
 (segment (start 138.1 110.62) (end 157.1 110.62) (width 0.2) (layer "F.Cu") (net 13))
 (segment (start 124.7775 85.56625) (end 137.33375 85.56625) (width 0.2) (layer "F.Cu") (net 19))
 (segment (start 137.33375 85.56625) (end 138 84.9) (width 0.2) (layer "F.Cu") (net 19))
 (segment (start 155.48375 104.61625) (end 157.1 103) (width 0.2) (layer "F.Cu") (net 20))
 (segment (start 143.8275 104.61625) (end 155.48375 104.61625) (width 0.2) (layer "F.Cu") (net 20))
 (segment (start 174.58375 104.61625) (end 176.2 103) (width 0.2) (layer "F.Cu") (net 11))
 (segment (start 162.8775 104.61625) (end 174.58375 104.61625) (width 0.2) (layer "F.Cu") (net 11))
 (segment (start 176.5 84.9) (end 174.64375 84.9) (width 0.2) (layer "F.Cu") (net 10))
 (segment (start 174.64375 84.9) (end 173.9375 85.60625) (width 0.2) (layer "F.Cu") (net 10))
 (segment (start 157.2 69.34) (end 120.7 69.34) (width 0.2) (layer "F.Cu") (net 16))
 (segment (start 164.56 61.98) (end 157.2 69.34) (width 0.2) (layer "F.Cu") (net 16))
 (segment (start 167.1 61.98) (end 167.1 60.90237) (width 0.2) (layer "F.Cu") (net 15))
 (segment (start 167.1 60.90237) (end 165.82563 59.628) (width 0.2) (layer "F.Cu") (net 15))
 (segment (start 121.177 66.8) (end 120.7 66.8) (width 0.2) (layer "F.Cu") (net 15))
 (segment (start 128.349 59.628) (end 121.177 66.8) (width 0.2) (layer "F.Cu") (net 15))
 (segment (start 165.82563 59.628) (end 128.349 59.628) (width 0.2) (layer "F.Cu") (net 15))
 (segment (start 171.117 86.377) (end 171.117 59.889374) (width 0.2) (layer "F.Cu") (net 5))
 (segment (start 144.5 98.7) (end 146.776251 100.976251) (width 0.2) (layer "F.Cu") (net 5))
 (segment (start 149.597186 103.47725) (end 154.01675 103.47725) (width 0.2) (layer "F.Cu") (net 5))
 (segment (start 171.378374 59.628) (end 172.981626 59.628) (width 0.2) (layer "F.Cu") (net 5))
 (segment (start 150.1775 83.0225) (end 150.2 83) (width 0.2) (layer "F.Cu") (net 5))
 (segment (start 150.1775 83.02625) (end 150.1775 83.0225) (width 0.2) (layer "F.Cu") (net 5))
 (segment (start 132.227499 100.976251) (end 147.096187 100.976251) (width 0.2) (layer "F.Cu") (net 5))
 (segment (start 171.117 59.889374) (end 171.378374 59.628) (width 0.2) (layer "F.Cu") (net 5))
 (segment (start 174.72 61.366374) (end 174.72 61.98) (width 0.2) (layer "F.Cu") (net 5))
 (segment (start 131.1275 102.07625) (end 132.227499 100.976251) (width 0.2) (layer "F.Cu") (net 5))
 (segment (start 172.981626 59.628) (end 174.72 61.366374) (width 0.2) (layer "F.Cu") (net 5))
 (segment (start 154.01675 103.47725) (end 171.117 86.377) (width 0.2) (layer "F.Cu") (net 5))
 (segment (start 147.096187 100.976251) (end 149.597186 103.47725) (width 0.2) (layer "F.Cu") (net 5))
 (segment (start 146.776251 100.976251) (end 147.096187 100.976251) (width 0.2) (layer "F.Cu") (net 5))
 (via (at 144.5 98.7) (size 0.6) (drill 0.3) (layers "F.Cu" "B.Cu") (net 5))
 (segment (start 150.2 93) (end 144.5 98.7) (width 0.2) (layer "B.Cu") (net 5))
 (segment (start 150.2 83) (end 150.2 93) (width 0.2) (layer "B.Cu") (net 5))
 (segment (start 177.26 61.98) (end 177.26 60.90237) (width 0.2) (layer "F.Cu") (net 12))
 (segment (start 131.1275 83.02625) (end 137.6833 83.02625) (width 0.2) (layer "F.Cu") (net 12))
 (segment (start 175.58463 59.227) (end 169.239374 59.227) (width 0.2) (layer "F.Cu") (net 12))
 (segment (start 177.26 60.90237) (end 175.58463 59.227) (width 0.2) (layer "F.Cu") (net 12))
 (segment (start 137.6833 83.02625) (end 141.3565 86.69945) (width 0.2) (layer "F.Cu") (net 12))
 (segment (start 141.4 86.65595) (end 141.3565 86.69945) (width 0.2) (layer "F.Cu") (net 12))
 (segment (start 141.3565 86.69945) (end 141.3565 93.25525) (width 0.2) (layer "F.Cu") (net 12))
 (segment (start 169.239374 59.227) (end 168.163 60.303374) (width 0.2) (layer "F.Cu") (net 12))
 (segment (start 143.03475 84.16525) (end 142.3 84.9) (width 0.2) (layer "F.Cu") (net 12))
 (segment (start 141.3565 93.25525) (end 150.1775 102.07625) (width 0.2) (layer "F.Cu") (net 12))
 (segment (start 146.41806 84.16525) (end 143.03475 84.16525) (width 0.2) (layer "F.Cu") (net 12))
 (segment (start 141.4 86.1) (end 141.4 86.65595) (width 0.2) (layer "F.Cu") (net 12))
 (segment (start 168.163 60.303374) (end 168.163 62.42031) (width 0.2) (layer "F.Cu") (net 12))
 (segment (start 168.163 62.42031) (end 146.41806 84.16525) (width 0.2) (layer "F.Cu") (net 12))
 (via (at 141.4 86.1) (size 0.6) (drill 0.3) (layers "F.Cu" "B.Cu") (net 12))
 (via (at 142.3 84.9) (size 0.6) (drill 0.3) (layers "F.Cu" "B.Cu") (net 12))
 (segment (start 142.3 84.9) (end 142.3 85.2) (width 0.2) (layer "B.Cu") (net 12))
 (segment (start 142.3 85.2) (end 141.4 86.1) (width 0.2) (layer "B.Cu") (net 12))
 (segment (start 169.2275 102.07625) (end 173.9375 97.36625) (width 0.2) (layer "F.Cu") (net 9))
 (segment (start 173.9375 90.60625) (end 172.1 88.76875) (width 0.2) (layer "F.Cu") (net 9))
 (segment (start 173.9375 97.36625) (end 173.9375 90.60625) (width 0.2) (layer "F.Cu") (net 9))
 (segment (start 172.1 88.76875) (end 172.1 80.4) (width 0.2) (layer "F.Cu") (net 9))
 (via (at 172.1 80.4) (size 0.6) (drill 0.3) (layers "F.Cu" "B.Cu") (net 9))
 (segment (start 172.1 80.4) (end 170.28 80.4) (width 0.2) (layer "B.Cu") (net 9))
 (segment (start 170.28 80.4) (end 167.1 77.22) (width 0.2) (layer "B.Cu") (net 9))
 (segment (start 159.4375 90.60625) (end 160.89375 90.60625) (width 0.2) (layer "F.Cu") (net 8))
 (segment (start 160.89375 90.60625) (end 161.7 89.8) (width 0.2) (layer "F.Cu") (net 8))
 (via (at 161.7 89.8) (size 0.6) (drill 0.3) (layers "F.Cu" "B.Cu") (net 8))
 (segment (start 161.7 89.8) (end 162.02 89.48) (width 0.2) (layer "B.Cu") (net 8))
 (segment (start 162.02 89.48) (end 162.02 77.22) (width 0.2) (layer "B.Cu") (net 8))
 (segment (start 159.4375 85.60625) (end 164.56 80.48375) (width 0.2) (layer "F.Cu") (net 7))
 (segment (start 164.56 80.48375) (end 164.56 77.22) (width 0.2) (layer "F.Cu") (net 7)))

